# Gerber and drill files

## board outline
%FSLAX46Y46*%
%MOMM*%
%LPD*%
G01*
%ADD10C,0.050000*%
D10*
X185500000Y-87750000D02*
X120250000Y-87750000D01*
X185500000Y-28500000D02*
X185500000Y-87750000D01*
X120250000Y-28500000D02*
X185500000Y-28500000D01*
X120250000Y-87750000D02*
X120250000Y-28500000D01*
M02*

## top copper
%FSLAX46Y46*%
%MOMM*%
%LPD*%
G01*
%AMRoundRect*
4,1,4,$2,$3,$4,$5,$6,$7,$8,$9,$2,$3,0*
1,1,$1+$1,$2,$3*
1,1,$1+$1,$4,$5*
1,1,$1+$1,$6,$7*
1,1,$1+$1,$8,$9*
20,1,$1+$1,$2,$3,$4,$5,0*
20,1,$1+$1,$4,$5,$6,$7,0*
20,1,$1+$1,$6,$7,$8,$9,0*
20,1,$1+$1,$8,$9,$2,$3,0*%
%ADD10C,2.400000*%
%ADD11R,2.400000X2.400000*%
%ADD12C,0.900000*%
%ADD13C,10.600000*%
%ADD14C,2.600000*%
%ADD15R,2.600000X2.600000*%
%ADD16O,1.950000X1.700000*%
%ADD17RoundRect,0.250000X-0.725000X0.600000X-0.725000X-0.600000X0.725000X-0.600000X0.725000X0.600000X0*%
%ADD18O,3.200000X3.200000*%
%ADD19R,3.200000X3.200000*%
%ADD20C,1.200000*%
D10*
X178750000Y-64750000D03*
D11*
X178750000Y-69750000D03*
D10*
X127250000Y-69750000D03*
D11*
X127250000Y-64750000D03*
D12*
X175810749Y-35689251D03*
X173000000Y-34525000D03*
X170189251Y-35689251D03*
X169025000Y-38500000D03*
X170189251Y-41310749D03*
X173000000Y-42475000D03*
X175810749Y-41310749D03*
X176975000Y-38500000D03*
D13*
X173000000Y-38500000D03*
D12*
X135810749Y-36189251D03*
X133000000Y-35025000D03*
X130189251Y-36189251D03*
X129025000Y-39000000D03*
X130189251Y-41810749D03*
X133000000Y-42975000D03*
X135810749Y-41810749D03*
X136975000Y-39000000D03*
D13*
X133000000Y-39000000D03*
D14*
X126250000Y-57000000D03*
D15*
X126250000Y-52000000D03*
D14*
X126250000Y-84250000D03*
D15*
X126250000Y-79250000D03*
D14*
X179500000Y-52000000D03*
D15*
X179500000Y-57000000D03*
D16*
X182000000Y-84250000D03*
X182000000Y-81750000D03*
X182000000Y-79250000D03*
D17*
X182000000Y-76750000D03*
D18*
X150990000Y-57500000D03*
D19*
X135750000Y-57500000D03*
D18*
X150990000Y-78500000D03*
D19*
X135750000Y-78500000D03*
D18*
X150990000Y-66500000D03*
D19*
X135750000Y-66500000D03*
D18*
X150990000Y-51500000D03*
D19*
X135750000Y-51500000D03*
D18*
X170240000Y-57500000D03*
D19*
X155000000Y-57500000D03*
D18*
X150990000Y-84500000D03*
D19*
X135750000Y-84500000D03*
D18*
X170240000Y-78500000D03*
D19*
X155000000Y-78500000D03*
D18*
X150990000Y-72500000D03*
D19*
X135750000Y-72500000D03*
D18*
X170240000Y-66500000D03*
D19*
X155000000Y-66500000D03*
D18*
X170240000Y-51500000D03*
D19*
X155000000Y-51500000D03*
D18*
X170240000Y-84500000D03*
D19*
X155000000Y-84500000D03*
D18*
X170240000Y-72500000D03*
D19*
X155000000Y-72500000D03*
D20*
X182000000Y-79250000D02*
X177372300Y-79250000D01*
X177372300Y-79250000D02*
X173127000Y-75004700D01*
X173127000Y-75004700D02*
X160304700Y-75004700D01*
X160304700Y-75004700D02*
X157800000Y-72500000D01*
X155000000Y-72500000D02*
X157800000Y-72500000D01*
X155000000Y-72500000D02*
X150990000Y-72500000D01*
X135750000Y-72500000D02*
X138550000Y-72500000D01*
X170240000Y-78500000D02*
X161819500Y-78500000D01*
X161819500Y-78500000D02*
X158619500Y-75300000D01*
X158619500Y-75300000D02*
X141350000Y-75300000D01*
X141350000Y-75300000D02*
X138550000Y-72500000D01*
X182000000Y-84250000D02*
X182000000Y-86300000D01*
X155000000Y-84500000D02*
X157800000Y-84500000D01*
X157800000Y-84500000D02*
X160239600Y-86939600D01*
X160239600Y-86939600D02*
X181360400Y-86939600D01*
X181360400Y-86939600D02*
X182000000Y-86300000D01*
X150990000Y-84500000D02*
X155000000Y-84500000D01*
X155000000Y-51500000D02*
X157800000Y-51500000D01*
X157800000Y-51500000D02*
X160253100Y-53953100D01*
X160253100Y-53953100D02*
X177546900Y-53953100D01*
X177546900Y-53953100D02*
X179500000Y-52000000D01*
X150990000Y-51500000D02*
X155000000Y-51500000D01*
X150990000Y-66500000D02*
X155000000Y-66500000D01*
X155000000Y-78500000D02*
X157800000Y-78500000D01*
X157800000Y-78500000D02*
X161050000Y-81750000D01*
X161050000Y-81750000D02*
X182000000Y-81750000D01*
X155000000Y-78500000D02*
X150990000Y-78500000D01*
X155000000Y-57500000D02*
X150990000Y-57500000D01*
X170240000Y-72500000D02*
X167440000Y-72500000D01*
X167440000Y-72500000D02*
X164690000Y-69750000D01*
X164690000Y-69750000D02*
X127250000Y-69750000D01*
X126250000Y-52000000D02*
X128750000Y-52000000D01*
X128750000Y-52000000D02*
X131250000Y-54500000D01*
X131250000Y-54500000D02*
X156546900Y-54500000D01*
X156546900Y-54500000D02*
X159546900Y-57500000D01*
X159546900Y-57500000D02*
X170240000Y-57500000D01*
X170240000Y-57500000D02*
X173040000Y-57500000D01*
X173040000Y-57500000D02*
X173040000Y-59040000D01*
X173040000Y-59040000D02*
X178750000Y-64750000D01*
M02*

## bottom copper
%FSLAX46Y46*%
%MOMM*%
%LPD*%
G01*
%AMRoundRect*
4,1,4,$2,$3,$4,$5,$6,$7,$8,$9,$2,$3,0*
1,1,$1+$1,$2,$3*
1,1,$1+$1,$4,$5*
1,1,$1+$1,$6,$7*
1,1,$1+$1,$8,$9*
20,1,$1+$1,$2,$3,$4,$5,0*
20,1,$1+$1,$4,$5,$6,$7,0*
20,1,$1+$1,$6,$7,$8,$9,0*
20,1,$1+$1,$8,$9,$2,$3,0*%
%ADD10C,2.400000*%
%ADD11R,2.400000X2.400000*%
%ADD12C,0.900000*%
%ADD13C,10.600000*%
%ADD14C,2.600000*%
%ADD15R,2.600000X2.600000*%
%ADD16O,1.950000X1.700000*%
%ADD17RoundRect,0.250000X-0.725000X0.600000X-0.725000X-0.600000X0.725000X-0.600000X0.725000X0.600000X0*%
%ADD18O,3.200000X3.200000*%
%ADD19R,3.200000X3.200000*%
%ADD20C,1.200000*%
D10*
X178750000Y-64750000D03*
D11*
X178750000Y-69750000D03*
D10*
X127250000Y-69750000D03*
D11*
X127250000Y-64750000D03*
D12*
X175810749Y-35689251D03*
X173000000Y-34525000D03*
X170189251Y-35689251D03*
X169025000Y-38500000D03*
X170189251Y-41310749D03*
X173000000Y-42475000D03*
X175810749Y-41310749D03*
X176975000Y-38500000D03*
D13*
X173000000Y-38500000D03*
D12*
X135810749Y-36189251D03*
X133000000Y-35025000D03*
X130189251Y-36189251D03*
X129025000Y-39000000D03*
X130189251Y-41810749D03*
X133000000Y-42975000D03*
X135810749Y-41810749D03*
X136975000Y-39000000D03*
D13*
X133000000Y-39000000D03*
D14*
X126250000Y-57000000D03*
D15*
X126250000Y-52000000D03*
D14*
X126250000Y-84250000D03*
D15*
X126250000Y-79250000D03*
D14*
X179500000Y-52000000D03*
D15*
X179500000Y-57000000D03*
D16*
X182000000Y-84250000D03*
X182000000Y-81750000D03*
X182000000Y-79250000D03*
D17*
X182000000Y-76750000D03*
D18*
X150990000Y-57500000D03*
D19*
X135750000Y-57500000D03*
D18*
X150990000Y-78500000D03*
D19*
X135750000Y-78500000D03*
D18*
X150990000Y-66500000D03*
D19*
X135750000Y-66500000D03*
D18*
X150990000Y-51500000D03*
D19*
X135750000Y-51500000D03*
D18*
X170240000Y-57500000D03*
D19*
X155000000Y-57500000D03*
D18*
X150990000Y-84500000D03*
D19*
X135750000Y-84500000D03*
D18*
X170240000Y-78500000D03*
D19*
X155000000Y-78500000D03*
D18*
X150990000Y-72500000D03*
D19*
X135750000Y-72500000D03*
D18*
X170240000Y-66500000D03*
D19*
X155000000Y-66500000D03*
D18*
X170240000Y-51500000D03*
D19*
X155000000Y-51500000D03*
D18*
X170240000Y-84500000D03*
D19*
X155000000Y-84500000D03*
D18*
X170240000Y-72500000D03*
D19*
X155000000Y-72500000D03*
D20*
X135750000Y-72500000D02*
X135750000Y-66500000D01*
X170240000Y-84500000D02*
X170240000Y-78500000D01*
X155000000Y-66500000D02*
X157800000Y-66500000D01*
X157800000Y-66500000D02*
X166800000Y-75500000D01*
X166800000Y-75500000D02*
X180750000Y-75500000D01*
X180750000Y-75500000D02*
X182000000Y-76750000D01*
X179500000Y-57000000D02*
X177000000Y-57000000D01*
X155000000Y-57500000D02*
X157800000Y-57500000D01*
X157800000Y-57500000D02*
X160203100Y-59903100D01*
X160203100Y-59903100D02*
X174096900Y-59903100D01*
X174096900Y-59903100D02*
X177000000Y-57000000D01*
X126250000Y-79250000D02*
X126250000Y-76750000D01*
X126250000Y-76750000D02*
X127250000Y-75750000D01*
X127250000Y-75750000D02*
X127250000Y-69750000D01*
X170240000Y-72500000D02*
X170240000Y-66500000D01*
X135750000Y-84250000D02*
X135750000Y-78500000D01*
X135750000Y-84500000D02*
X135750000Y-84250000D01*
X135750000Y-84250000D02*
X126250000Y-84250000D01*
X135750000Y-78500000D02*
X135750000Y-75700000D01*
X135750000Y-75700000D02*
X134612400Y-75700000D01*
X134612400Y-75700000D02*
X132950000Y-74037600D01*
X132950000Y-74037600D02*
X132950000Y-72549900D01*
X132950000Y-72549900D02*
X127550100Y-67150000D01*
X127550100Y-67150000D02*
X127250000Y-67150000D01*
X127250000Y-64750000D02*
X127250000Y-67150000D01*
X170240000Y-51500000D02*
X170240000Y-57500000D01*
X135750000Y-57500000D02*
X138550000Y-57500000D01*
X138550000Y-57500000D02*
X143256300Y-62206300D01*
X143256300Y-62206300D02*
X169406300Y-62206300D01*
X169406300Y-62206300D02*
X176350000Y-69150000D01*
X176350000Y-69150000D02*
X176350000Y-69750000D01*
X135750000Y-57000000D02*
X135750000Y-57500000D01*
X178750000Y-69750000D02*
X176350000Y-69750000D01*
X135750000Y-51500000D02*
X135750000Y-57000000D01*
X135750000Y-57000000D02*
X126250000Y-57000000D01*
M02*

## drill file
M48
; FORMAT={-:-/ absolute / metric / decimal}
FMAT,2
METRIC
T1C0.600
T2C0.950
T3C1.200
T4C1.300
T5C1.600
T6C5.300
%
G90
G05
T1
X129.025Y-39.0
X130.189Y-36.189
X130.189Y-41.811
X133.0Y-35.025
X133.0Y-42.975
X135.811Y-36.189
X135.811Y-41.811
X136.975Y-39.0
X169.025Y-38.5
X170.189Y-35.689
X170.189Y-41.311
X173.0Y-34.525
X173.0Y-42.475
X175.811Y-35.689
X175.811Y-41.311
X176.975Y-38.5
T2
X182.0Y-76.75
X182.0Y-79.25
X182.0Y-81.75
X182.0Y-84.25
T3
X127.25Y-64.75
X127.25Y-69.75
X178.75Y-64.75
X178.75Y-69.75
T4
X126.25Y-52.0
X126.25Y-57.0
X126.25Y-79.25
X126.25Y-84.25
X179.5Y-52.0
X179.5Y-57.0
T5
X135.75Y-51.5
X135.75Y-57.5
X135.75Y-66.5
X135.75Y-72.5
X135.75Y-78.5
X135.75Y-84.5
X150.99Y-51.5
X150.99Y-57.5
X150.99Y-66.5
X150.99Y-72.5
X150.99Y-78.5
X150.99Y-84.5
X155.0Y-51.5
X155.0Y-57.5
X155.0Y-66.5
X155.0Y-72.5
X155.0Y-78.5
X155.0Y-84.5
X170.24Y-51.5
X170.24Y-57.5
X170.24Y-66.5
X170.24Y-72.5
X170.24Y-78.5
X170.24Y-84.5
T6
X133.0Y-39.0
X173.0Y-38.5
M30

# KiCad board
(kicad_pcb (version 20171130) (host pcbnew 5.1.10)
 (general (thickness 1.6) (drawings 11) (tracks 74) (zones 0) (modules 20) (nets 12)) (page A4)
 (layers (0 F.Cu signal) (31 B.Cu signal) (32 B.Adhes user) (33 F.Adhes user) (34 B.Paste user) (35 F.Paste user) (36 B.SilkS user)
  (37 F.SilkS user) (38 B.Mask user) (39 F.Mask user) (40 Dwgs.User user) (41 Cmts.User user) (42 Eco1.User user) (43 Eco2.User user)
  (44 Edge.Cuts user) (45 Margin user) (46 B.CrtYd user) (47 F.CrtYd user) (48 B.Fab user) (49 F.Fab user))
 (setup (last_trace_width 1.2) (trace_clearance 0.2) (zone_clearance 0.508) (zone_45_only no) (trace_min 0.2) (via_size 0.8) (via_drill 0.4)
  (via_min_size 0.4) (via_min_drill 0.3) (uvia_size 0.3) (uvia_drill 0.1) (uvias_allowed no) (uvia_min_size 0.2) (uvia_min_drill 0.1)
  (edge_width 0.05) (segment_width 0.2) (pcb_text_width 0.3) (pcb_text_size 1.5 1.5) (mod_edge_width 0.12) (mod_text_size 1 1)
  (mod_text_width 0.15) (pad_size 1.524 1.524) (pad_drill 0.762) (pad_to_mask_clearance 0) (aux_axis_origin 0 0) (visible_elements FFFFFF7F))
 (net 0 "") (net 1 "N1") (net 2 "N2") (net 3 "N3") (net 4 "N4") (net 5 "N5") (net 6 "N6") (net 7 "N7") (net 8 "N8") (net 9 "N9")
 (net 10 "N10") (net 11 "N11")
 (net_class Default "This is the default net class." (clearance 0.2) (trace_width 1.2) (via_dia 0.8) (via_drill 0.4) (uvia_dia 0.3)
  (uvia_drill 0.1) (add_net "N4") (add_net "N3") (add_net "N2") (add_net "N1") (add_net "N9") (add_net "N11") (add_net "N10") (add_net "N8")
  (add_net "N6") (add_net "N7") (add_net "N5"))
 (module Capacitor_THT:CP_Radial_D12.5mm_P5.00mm (layer F.Cu) (at 178.75 69.75 90)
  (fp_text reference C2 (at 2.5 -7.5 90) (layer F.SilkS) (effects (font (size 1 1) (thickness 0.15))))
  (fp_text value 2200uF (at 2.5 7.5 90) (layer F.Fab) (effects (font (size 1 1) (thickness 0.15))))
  (pad 2 thru_hole circle (at 5 0 90) (size 2.4 2.4) (drill 1.2) (layers *.Cu *.Mask) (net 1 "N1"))
  (pad 1 thru_hole rect (at 0 0 90) (size 2.4 2.4) (drill 1.2) (layers *.Cu *.Mask) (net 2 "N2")))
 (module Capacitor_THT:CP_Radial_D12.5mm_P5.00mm (layer F.Cu) (at 127.25 64.75 270)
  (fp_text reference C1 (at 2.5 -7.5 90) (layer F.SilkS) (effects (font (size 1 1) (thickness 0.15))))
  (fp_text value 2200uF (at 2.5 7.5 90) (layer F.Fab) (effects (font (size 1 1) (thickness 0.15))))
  (pad 2 thru_hole circle (at 5 0 270) (size 2.4 2.4) (drill 1.2) (layers *.Cu *.Mask) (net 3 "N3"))
  (pad 1 thru_hole rect (at 0 0 270) (size 2.4 2.4) (drill 1.2) (layers *.Cu *.Mask) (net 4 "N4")))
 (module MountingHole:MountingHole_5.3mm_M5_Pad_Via (layer F.Cu) (at 173 38.5)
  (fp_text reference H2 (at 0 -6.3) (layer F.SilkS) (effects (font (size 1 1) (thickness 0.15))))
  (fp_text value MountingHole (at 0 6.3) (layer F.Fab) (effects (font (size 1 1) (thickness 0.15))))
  (pad 1 thru_hole circle (at 2.810749 -2.810749) (size 0.9 0.9) (drill 0.6) (layers *.Cu *.Mask))
  (pad 1 thru_hole circle (at 0 -3.975) (size 0.9 0.9) (drill 0.6) (layers *.Cu *.Mask))
  (pad 1 thru_hole circle (at -2.810749 -2.810749) (size 0.9 0.9) (drill 0.6) (layers *.Cu *.Mask))
  (pad 1 thru_hole circle (at -3.975 0) (size 0.9 0.9) (drill 0.6) (layers *.Cu *.Mask))
  (pad 1 thru_hole circle (at -2.810749 2.810749) (size 0.9 0.9) (drill 0.6) (layers *.Cu *.Mask))
  (pad 1 thru_hole circle (at 0 3.975) (size 0.9 0.9) (drill 0.6) (layers *.Cu *.Mask))
  (pad 1 thru_hole circle (at 2.810749 2.810749) (size 0.9 0.9) (drill 0.6) (layers *.Cu *.Mask))
  (pad 1 thru_hole circle (at 3.975 0) (size 0.9 0.9) (drill 0.6) (layers *.Cu *.Mask))
  (pad 1 thru_hole circle (at 0 0) (size 10.6 10.6) (drill 5.3) (layers *.Cu *.Mask)))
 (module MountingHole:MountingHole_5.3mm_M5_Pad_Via (layer F.Cu) (at 133 39)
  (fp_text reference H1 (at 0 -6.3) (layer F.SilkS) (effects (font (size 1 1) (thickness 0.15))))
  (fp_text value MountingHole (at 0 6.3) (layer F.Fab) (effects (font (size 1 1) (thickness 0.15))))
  (pad 1 thru_hole circle (at 2.810749 -2.810749) (size 0.9 0.9) (drill 0.6) (layers *.Cu *.Mask))
  (pad 1 thru_hole circle (at 0 -3.975) (size 0.9 0.9) (drill 0.6) (layers *.Cu *.Mask))
  (pad 1 thru_hole circle (at -2.810749 -2.810749) (size 0.9 0.9) (drill 0.6) (layers *.Cu *.Mask))
  (pad 1 thru_hole circle (at -3.975 0) (size 0.9 0.9) (drill 0.6) (layers *.Cu *.Mask))
  (pad 1 thru_hole circle (at -2.810749 2.810749) (size 0.9 0.9) (drill 0.6) (layers *.Cu *.Mask))
  (pad 1 thru_hole circle (at 0 3.975) (size 0.9 0.9) (drill 0.6) (layers *.Cu *.Mask))
  (pad 1 thru_hole circle (at 2.810749 2.810749) (size 0.9 0.9) (drill 0.6) (layers *.Cu *.Mask))
  (pad 1 thru_hole circle (at 3.975 0) (size 0.9 0.9) (drill 0.6) (layers *.Cu *.Mask))
  (pad 1 thru_hole circle (at 0 0) (size 10.6 10.6) (drill 5.3) (layers *.Cu *.Mask)))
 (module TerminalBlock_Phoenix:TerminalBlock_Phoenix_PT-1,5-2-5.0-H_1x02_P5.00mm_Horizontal (layer F.Cu) (at 126.25 52 270)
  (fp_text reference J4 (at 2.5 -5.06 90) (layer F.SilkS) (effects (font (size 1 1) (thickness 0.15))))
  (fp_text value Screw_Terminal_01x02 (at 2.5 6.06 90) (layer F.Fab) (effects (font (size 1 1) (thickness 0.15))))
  (pad 2 thru_hole circle (at 5 0 270) (size 2.6 2.6) (drill 1.3) (layers *.Cu *.Mask) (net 2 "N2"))
  (pad 1 thru_hole rect (at 0 0 270) (size 2.6 2.6) (drill 1.3) (layers *.Cu *.Mask) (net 1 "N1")))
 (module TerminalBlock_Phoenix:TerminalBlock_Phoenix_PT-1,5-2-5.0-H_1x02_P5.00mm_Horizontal (layer F.Cu) (at 126.25 79.25 270)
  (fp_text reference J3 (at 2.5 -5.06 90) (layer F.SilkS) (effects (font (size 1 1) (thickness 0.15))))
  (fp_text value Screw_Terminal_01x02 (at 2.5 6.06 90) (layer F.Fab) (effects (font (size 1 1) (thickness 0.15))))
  (pad 2 thru_hole circle (at 5 0 270) (size 2.6 2.6) (drill 1.3) (layers *.Cu *.Mask) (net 4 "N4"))
  (pad 1 thru_hole rect (at 0 0 270) (size 2.6 2.6) (drill 1.3) (layers *.Cu *.Mask) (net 3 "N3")))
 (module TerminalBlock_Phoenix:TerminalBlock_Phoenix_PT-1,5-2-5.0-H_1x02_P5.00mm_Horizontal (layer F.Cu) (at 179.5 57 90)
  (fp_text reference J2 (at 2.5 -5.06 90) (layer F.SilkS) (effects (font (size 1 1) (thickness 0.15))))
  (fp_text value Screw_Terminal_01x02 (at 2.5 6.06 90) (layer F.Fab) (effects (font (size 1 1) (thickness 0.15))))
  (pad 2 thru_hole circle (at 5 0 90) (size 2.6 2.6) (drill 1.3) (layers *.Cu *.Mask) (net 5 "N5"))
  (pad 1 thru_hole rect (at 0 0 90) (size 2.6 2.6) (drill 1.3) (layers *.Cu *.Mask) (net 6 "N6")))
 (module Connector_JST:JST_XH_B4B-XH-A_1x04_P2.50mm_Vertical (layer F.Cu) (at 182 76.75 270)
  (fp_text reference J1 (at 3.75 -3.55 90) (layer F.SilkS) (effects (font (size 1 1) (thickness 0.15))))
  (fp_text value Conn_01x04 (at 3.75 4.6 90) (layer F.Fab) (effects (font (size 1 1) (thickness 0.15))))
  (pad 4 thru_hole oval (at 7.5 0 270) (size 1.7 1.95) (drill 0.95) (layers *.Cu *.Mask) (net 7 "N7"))
  (pad 3 thru_hole oval (at 5 0 270) (size 1.7 1.95) (drill 0.95) (layers *.Cu *.Mask) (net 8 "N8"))
  (pad 2 thru_hole oval (at 2.5 0 270) (size 1.7 1.95) (drill 0.95) (layers *.Cu *.Mask) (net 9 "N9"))
  (pad 1 thru_hole roundrect (at 0 0 270) (size 1.7 1.95) (drill 0.95) (layers *.Cu *.Mask) (roundrect_rratio 0.1470588235294118)
   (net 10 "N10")))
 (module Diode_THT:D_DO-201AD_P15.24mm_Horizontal (layer F.Cu) (at 135.75 57.5)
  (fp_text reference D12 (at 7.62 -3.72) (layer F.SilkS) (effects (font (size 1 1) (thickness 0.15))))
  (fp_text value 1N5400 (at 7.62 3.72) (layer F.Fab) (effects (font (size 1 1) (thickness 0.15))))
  (pad 2 thru_hole oval (at 15.24 0) (size 3.2 3.2) (drill 1.6) (layers *.Cu *.Mask) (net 6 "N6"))
  (pad 1 thru_hole rect (at 0 0) (size 3.2 3.2) (drill 1.6) (layers *.Cu *.Mask) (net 2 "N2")))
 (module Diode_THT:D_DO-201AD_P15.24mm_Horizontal (layer F.Cu) (at 135.75 78.5)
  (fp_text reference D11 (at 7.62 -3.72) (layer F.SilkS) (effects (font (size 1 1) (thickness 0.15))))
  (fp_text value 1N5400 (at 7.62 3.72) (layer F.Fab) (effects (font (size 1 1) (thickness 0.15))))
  (pad 2 thru_hole oval (at 15.24 0) (size 3.2 3.2) (drill 1.6) (layers *.Cu *.Mask) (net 8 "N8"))
  (pad 1 thru_hole rect (at 0 0) (size 3.2 3.2) (drill 1.6) (layers *.Cu *.Mask) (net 4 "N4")))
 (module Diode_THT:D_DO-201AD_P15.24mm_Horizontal (layer F.Cu) (at 135.75 66.5)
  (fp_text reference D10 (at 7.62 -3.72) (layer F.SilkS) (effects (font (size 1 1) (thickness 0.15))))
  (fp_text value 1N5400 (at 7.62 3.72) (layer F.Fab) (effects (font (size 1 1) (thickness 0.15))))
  (pad 2 thru_hole oval (at 15.24 0) (size 3.2 3.2) (drill 1.6) (layers *.Cu *.Mask) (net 10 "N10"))
  (pad 1 thru_hole rect (at 0 0) (size 3.2 3.2) (drill 1.6) (layers *.Cu *.Mask) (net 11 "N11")))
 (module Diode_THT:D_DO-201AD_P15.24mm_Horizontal (layer F.Cu) (at 135.75 51.5)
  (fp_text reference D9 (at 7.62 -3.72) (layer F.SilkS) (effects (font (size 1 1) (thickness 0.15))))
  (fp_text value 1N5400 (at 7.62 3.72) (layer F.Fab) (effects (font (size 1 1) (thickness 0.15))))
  (pad 2 thru_hole oval (at 15.24 0) (size 3.2 3.2) (drill 1.6) (layers *.Cu *.Mask) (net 5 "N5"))
  (pad 1 thru_hole rect (at 0 0) (size 3.2 3.2) (drill 1.6) (layers *.Cu *.Mask) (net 2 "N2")))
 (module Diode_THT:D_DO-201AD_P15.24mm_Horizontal (layer F.Cu) (at 155 57.5)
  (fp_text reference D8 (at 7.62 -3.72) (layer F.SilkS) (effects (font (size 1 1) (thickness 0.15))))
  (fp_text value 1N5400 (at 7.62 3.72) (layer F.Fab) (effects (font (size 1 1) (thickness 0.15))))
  (pad 2 thru_hole oval (at 15.24 0) (size 3.2 3.2) (drill 1.6) (layers *.Cu *.Mask) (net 1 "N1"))
  (pad 1 thru_hole rect (at 0 0) (size 3.2 3.2) (drill 1.6) (layers *.Cu *.Mask) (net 6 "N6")))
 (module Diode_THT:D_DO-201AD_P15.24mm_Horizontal (layer F.Cu) (at 135.75 84.5)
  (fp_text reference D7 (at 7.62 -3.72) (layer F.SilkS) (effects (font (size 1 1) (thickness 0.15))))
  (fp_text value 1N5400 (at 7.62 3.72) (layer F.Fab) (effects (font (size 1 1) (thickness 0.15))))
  (pad 2 thru_hole oval (at 15.24 0) (size 3.2 3.2) (drill 1.6) (layers *.Cu *.Mask) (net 7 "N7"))
  (pad 1 thru_hole rect (at 0 0) (size 3.2 3.2) (drill 1.6) (layers *.Cu *.Mask) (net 4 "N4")))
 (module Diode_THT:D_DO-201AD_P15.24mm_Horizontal (layer F.Cu) (at 155 78.5)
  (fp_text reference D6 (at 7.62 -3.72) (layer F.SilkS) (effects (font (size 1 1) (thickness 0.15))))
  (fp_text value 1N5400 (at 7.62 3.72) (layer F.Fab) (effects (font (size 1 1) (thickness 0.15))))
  (pad 2 thru_hole oval (at 15.24 0) (size 3.2 3.2) (drill 1.6) (layers *.Cu *.Mask) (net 11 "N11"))
  (pad 1 thru_hole rect (at 0 0) (size 3.2 3.2) (drill 1.6) (layers *.Cu *.Mask) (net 8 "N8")))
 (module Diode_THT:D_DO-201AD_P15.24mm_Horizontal (layer F.Cu) (at 135.75 72.5)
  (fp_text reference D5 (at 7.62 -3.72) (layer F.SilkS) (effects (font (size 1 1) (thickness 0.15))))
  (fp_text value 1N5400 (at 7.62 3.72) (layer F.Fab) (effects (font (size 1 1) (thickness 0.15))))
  (pad 2 thru_hole oval (at 15.24 0) (size 3.2 3.2) (drill 1.6) (layers *.Cu *.Mask) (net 9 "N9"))
  (pad 1 thru_hole rect (at 0 0) (size 3.2 3.2) (drill 1.6) (layers *.Cu *.Mask) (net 11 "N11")))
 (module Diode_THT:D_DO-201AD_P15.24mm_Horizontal (layer F.Cu) (at 155 66.5)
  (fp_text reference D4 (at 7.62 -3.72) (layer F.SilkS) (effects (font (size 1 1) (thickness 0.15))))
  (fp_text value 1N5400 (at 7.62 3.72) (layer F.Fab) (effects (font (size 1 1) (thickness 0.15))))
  (pad 2 thru_hole oval (at 15.24 0) (size 3.2 3.2) (drill 1.6) (layers *.Cu *.Mask) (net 3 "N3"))
  (pad 1 thru_hole rect (at 0 0) (size 3.2 3.2) (drill 1.6) (layers *.Cu *.Mask) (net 10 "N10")))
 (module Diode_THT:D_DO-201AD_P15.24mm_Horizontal (layer F.Cu) (at 155 51.5)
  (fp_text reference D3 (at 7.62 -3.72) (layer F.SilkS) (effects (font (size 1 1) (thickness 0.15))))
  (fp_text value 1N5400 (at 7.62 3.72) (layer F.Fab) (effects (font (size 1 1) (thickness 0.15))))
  (pad 2 thru_hole oval (at 15.24 0) (size 3.2 3.2) (drill 1.6) (layers *.Cu *.Mask) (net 1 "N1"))
  (pad 1 thru_hole rect (at 0 0) (size 3.2 3.2) (drill 1.6) (layers *.Cu *.Mask) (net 5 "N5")))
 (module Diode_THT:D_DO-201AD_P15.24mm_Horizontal (layer F.Cu) (at 155 84.5)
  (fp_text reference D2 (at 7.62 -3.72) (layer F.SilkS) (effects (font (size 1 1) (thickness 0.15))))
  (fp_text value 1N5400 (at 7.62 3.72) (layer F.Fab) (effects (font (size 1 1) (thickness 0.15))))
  (pad 2 thru_hole oval (at 15.24 0) (size 3.2 3.2) (drill 1.6) (layers *.Cu *.Mask) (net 11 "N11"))
  (pad 1 thru_hole rect (at 0 0) (size 3.2 3.2) (drill 1.6) (layers *.Cu *.Mask) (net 7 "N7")))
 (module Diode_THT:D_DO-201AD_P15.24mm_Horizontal (layer F.Cu) (at 155 72.5)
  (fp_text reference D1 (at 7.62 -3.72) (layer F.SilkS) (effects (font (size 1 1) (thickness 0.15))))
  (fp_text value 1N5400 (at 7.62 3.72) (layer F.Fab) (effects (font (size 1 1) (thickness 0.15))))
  (pad 2 thru_hole oval (at 15.24 0) (size 3.2 3.2) (drill 1.6) (layers *.Cu *.Mask) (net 3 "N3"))
  (pad 1 thru_hole rect (at 0 0) (size 3.2 3.2) (drill 1.6) (layers *.Cu *.Mask) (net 9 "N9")))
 (gr_line (start 185.5 87.75) (end 120.25 87.75) (layer Edge.Cuts) (width 0.05))
 (gr_line (start 185.5 28.5) (end 185.5 87.75) (layer Edge.Cuts) (width 0.05))
 (gr_line (start 120.25 28.5) (end 185.5 28.5) (layer Edge.Cuts) (width 0.05))
 (gr_line (start 120.25 87.75) (end 120.25 28.5) (layer Edge.Cuts) (width 0.05))
 (segment (start 182 79.25) (end 177.3723 79.25) (width 1.2) (layer F.Cu) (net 9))
 (segment (start 177.3723 79.25) (end 173.127 75.0047) (width 1.2) (layer F.Cu) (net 9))
 (segment (start 173.127 75.0047) (end 160.3047 75.0047) (width 1.2) (layer F.Cu) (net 9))
 (segment (start 160.3047 75.0047) (end 157.8 72.5) (width 1.2) (layer F.Cu) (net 9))
 (segment (start 155 72.5) (end 157.8 72.5) (width 1.2) (layer F.Cu) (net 9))
 (segment (start 155 72.5) (end 150.99 72.5) (width 1.2) (layer F.Cu) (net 9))
 (segment (start 135.75 72.5) (end 138.55 72.5) (width 1.2) (layer F.Cu) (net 11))
 (segment (start 170.24 78.5) (end 161.8195 78.5) (width 1.2) (layer F.Cu) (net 11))
 (segment (start 161.8195 78.5) (end 158.6195 75.3) (width 1.2) (layer F.Cu) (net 11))
 (segment (start 158.6195 75.3) (end 141.35 75.3) (width 1.2) (layer F.Cu) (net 11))
 (segment (start 141.35 75.3) (end 138.55 72.5) (width 1.2) (layer F.Cu) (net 11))
 (segment (start 135.75 72.5) (end 135.75 66.5) (width 1.2) (layer B.Cu) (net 11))
 (segment (start 170.24 84.5) (end 170.24 78.5) (width 1.2) (layer B.Cu) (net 11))
 (segment (start 182 84.25) (end 182 86.3) (width 1.2) (layer F.Cu) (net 7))
 (segment (start 155 84.5) (end 157.8 84.5) (width 1.2) (layer F.Cu) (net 7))
 (segment (start 157.8 84.5) (end 160.2396 86.9396) (width 1.2) (layer F.Cu) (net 7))
 (segment (start 160.2396 86.9396) (end 181.3604 86.9396) (width 1.2) (layer F.Cu) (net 7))
 (segment (start 181.3604 86.9396) (end 182 86.3) (width 1.2) (layer F.Cu) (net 7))
 (segment (start 150.99 84.5) (end 155 84.5) (width 1.2) (layer F.Cu) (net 7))
 (segment (start 155 51.5) (end 157.8 51.5) (width 1.2) (layer F.Cu) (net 5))
 (segment (start 157.8 51.5) (end 160.2531 53.9531) (width 1.2) (layer F.Cu) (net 5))
 (segment (start 160.2531 53.9531) (end 177.5469 53.9531) (width 1.2) (layer F.Cu) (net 5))
 (segment (start 177.5469 53.9531) (end 179.5 52) (width 1.2) (layer F.Cu) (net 5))
 (segment (start 150.99 51.5) (end 155 51.5) (width 1.2) (layer F.Cu) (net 5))
 (segment (start 155 66.5) (end 157.8 66.5) (width 1.2) (layer B.Cu) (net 10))
 (segment (start 157.8 66.5) (end 166.8 75.5) (width 1.2) (layer B.Cu) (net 10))
 (segment (start 166.8 75.5) (end 180.75 75.5) (width 1.2) (layer B.Cu) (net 10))
 (segment (start 180.75 75.5) (end 182 76.75) (width 1.2) (layer B.Cu) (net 10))
 (segment (start 150.99 66.5) (end 155 66.5) (width 1.2) (layer F.Cu) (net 10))
 (segment (start 155 78.5) (end 157.8 78.5) (width 1.2) (layer F.Cu) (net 8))
 (segment (start 157.8 78.5) (end 161.05 81.75) (width 1.2) (layer F.Cu) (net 8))
 (segment (start 161.05 81.75) (end 182 81.75) (width 1.2) (layer F.Cu) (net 8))
 (segment (start 155 78.5) (end 150.99 78.5) (width 1.2) (layer F.Cu) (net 8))
 (segment (start 179.5 57) (end 177 57) (width 1.2) (layer B.Cu) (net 6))
 (segment (start 155 57.5) (end 157.8 57.5) (width 1.2) (layer B.Cu) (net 6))
 (segment (start 157.8 57.5) (end 160.2031 59.9031) (width 1.2) (layer B.Cu) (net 6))
 (segment (start 160.2031 59.9031) (end 174.0969 59.9031) (width 1.2) (layer B.Cu) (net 6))
 (segment (start 174.0969 59.9031) (end 177 57) (width 1.2) (layer B.Cu) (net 6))
 (segment (start 155 57.5) (end 150.99 57.5) (width 1.2) (layer F.Cu) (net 6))
 (segment (start 126.25 79.25) (end 126.25 76.75) (width 1.2) (layer B.Cu) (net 3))
 (segment (start 126.25 76.75) (end 127.25 75.75) (width 1.2) (layer B.Cu) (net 3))
 (segment (start 127.25 75.75) (end 127.25 69.75) (width 1.2) (layer B.Cu) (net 3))
 (segment (start 170.24 72.5) (end 167.44 72.5) (width 1.2) (layer F.Cu) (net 3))
 (segment (start 167.44 72.5) (end 164.69 69.75) (width 1.2) (layer F.Cu) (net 3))
 (segment (start 164.69 69.75) (end 127.25 69.75) (width 1.2) (layer F.Cu) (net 3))
 (segment (start 170.24 72.5) (end 170.24 66.5) (width 1.2) (layer B.Cu) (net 3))
 (segment (start 135.75 84.25) (end 135.75 78.5) (width 1.2) (layer B.Cu) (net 4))
 (segment (start 135.75 84.5) (end 135.75 84.25) (width 1.2) (layer B.Cu) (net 4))
 (segment (start 135.75 84.25) (end 126.25 84.25) (width 1.2) (layer B.Cu) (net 4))
 (segment (start 135.75 78.5) (end 135.75 75.7) (width 1.2) (layer B.Cu) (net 4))
 (segment (start 135.75 75.7) (end 134.6124 75.7) (width 1.2) (layer B.Cu) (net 4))
 (segment (start 134.6124 75.7) (end 132.95 74.0376) (width 1.2) (layer B.Cu) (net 4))
 (segment (start 132.95 74.0376) (end 132.95 72.5499) (width 1.2) (layer B.Cu) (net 4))
 (segment (start 132.95 72.5499) (end 127.5501 67.15) (width 1.2) (layer B.Cu) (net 4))
 (segment (start 127.5501 67.15) (end 127.25 67.15) (width 1.2) (layer B.Cu) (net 4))
 (segment (start 127.25 64.75) (end 127.25 67.15) (width 1.2) (layer B.Cu) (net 4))
 (segment (start 126.25 52) (end 128.75 52) (width 1.2) (layer F.Cu) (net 1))
 (segment (start 128.75 52) (end 131.25 54.5) (width 1.2) (layer F.Cu) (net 1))
 (segment (start 131.25 54.5) (end 156.5469 54.5) (width 1.2) (layer F.Cu) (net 1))
 (segment (start 156.5469 54.5) (end 159.5469 57.5) (width 1.2) (layer F.Cu) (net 1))
 (segment (start 159.5469 57.5) (end 170.24 57.5) (width 1.2) (layer F.Cu) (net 1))
 (segment (start 170.24 57.5) (end 173.04 57.5) (width 1.2) (layer F.Cu) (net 1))
 (segment (start 173.04 57.5) (end 173.04 59.04) (width 1.2) (layer F.Cu) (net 1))
 (segment (start 173.04 59.04) (end 178.75 64.75) (width 1.2) (layer F.Cu) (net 1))
 (segment (start 170.24 51.5) (end 170.24 57.5) (width 1.2) (layer B.Cu) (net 1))
 (segment (start 135.75 57.5) (end 138.55 57.5) (width 1.2) (layer B.Cu) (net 2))
 (segment (start 138.55 57.5) (end 143.2563 62.2063) (width 1.2) (layer B.Cu) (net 2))
 (segment (start 143.2563 62.2063) (end 169.4063 62.2063) (width 1.2) (layer B.Cu) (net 2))
 (segment (start 169.4063 62.2063) (end 176.35 69.15) (width 1.2) (layer B.Cu) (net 2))
 (segment (start 176.35 69.15) (end 176.35 69.75) (width 1.2) (layer B.Cu) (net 2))
 (segment (start 135.75 57) (end 135.75 57.5) (width 1.2) (layer B.Cu) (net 2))
 (segment (start 178.75 69.75) (end 176.35 69.75) (width 1.2) (layer B.Cu) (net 2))
 (segment (start 135.75 51.5) (end 135.75 57) (width 1.2) (layer B.Cu) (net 2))
 (segment (start 135.75 57) (end 126.25 57) (width 1.2) (layer B.Cu) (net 2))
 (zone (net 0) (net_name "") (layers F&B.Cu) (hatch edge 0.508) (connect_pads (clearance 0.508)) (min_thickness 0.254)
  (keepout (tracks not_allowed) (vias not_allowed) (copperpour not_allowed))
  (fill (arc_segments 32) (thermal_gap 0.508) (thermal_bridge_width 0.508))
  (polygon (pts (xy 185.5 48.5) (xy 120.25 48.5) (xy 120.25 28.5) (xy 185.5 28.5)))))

